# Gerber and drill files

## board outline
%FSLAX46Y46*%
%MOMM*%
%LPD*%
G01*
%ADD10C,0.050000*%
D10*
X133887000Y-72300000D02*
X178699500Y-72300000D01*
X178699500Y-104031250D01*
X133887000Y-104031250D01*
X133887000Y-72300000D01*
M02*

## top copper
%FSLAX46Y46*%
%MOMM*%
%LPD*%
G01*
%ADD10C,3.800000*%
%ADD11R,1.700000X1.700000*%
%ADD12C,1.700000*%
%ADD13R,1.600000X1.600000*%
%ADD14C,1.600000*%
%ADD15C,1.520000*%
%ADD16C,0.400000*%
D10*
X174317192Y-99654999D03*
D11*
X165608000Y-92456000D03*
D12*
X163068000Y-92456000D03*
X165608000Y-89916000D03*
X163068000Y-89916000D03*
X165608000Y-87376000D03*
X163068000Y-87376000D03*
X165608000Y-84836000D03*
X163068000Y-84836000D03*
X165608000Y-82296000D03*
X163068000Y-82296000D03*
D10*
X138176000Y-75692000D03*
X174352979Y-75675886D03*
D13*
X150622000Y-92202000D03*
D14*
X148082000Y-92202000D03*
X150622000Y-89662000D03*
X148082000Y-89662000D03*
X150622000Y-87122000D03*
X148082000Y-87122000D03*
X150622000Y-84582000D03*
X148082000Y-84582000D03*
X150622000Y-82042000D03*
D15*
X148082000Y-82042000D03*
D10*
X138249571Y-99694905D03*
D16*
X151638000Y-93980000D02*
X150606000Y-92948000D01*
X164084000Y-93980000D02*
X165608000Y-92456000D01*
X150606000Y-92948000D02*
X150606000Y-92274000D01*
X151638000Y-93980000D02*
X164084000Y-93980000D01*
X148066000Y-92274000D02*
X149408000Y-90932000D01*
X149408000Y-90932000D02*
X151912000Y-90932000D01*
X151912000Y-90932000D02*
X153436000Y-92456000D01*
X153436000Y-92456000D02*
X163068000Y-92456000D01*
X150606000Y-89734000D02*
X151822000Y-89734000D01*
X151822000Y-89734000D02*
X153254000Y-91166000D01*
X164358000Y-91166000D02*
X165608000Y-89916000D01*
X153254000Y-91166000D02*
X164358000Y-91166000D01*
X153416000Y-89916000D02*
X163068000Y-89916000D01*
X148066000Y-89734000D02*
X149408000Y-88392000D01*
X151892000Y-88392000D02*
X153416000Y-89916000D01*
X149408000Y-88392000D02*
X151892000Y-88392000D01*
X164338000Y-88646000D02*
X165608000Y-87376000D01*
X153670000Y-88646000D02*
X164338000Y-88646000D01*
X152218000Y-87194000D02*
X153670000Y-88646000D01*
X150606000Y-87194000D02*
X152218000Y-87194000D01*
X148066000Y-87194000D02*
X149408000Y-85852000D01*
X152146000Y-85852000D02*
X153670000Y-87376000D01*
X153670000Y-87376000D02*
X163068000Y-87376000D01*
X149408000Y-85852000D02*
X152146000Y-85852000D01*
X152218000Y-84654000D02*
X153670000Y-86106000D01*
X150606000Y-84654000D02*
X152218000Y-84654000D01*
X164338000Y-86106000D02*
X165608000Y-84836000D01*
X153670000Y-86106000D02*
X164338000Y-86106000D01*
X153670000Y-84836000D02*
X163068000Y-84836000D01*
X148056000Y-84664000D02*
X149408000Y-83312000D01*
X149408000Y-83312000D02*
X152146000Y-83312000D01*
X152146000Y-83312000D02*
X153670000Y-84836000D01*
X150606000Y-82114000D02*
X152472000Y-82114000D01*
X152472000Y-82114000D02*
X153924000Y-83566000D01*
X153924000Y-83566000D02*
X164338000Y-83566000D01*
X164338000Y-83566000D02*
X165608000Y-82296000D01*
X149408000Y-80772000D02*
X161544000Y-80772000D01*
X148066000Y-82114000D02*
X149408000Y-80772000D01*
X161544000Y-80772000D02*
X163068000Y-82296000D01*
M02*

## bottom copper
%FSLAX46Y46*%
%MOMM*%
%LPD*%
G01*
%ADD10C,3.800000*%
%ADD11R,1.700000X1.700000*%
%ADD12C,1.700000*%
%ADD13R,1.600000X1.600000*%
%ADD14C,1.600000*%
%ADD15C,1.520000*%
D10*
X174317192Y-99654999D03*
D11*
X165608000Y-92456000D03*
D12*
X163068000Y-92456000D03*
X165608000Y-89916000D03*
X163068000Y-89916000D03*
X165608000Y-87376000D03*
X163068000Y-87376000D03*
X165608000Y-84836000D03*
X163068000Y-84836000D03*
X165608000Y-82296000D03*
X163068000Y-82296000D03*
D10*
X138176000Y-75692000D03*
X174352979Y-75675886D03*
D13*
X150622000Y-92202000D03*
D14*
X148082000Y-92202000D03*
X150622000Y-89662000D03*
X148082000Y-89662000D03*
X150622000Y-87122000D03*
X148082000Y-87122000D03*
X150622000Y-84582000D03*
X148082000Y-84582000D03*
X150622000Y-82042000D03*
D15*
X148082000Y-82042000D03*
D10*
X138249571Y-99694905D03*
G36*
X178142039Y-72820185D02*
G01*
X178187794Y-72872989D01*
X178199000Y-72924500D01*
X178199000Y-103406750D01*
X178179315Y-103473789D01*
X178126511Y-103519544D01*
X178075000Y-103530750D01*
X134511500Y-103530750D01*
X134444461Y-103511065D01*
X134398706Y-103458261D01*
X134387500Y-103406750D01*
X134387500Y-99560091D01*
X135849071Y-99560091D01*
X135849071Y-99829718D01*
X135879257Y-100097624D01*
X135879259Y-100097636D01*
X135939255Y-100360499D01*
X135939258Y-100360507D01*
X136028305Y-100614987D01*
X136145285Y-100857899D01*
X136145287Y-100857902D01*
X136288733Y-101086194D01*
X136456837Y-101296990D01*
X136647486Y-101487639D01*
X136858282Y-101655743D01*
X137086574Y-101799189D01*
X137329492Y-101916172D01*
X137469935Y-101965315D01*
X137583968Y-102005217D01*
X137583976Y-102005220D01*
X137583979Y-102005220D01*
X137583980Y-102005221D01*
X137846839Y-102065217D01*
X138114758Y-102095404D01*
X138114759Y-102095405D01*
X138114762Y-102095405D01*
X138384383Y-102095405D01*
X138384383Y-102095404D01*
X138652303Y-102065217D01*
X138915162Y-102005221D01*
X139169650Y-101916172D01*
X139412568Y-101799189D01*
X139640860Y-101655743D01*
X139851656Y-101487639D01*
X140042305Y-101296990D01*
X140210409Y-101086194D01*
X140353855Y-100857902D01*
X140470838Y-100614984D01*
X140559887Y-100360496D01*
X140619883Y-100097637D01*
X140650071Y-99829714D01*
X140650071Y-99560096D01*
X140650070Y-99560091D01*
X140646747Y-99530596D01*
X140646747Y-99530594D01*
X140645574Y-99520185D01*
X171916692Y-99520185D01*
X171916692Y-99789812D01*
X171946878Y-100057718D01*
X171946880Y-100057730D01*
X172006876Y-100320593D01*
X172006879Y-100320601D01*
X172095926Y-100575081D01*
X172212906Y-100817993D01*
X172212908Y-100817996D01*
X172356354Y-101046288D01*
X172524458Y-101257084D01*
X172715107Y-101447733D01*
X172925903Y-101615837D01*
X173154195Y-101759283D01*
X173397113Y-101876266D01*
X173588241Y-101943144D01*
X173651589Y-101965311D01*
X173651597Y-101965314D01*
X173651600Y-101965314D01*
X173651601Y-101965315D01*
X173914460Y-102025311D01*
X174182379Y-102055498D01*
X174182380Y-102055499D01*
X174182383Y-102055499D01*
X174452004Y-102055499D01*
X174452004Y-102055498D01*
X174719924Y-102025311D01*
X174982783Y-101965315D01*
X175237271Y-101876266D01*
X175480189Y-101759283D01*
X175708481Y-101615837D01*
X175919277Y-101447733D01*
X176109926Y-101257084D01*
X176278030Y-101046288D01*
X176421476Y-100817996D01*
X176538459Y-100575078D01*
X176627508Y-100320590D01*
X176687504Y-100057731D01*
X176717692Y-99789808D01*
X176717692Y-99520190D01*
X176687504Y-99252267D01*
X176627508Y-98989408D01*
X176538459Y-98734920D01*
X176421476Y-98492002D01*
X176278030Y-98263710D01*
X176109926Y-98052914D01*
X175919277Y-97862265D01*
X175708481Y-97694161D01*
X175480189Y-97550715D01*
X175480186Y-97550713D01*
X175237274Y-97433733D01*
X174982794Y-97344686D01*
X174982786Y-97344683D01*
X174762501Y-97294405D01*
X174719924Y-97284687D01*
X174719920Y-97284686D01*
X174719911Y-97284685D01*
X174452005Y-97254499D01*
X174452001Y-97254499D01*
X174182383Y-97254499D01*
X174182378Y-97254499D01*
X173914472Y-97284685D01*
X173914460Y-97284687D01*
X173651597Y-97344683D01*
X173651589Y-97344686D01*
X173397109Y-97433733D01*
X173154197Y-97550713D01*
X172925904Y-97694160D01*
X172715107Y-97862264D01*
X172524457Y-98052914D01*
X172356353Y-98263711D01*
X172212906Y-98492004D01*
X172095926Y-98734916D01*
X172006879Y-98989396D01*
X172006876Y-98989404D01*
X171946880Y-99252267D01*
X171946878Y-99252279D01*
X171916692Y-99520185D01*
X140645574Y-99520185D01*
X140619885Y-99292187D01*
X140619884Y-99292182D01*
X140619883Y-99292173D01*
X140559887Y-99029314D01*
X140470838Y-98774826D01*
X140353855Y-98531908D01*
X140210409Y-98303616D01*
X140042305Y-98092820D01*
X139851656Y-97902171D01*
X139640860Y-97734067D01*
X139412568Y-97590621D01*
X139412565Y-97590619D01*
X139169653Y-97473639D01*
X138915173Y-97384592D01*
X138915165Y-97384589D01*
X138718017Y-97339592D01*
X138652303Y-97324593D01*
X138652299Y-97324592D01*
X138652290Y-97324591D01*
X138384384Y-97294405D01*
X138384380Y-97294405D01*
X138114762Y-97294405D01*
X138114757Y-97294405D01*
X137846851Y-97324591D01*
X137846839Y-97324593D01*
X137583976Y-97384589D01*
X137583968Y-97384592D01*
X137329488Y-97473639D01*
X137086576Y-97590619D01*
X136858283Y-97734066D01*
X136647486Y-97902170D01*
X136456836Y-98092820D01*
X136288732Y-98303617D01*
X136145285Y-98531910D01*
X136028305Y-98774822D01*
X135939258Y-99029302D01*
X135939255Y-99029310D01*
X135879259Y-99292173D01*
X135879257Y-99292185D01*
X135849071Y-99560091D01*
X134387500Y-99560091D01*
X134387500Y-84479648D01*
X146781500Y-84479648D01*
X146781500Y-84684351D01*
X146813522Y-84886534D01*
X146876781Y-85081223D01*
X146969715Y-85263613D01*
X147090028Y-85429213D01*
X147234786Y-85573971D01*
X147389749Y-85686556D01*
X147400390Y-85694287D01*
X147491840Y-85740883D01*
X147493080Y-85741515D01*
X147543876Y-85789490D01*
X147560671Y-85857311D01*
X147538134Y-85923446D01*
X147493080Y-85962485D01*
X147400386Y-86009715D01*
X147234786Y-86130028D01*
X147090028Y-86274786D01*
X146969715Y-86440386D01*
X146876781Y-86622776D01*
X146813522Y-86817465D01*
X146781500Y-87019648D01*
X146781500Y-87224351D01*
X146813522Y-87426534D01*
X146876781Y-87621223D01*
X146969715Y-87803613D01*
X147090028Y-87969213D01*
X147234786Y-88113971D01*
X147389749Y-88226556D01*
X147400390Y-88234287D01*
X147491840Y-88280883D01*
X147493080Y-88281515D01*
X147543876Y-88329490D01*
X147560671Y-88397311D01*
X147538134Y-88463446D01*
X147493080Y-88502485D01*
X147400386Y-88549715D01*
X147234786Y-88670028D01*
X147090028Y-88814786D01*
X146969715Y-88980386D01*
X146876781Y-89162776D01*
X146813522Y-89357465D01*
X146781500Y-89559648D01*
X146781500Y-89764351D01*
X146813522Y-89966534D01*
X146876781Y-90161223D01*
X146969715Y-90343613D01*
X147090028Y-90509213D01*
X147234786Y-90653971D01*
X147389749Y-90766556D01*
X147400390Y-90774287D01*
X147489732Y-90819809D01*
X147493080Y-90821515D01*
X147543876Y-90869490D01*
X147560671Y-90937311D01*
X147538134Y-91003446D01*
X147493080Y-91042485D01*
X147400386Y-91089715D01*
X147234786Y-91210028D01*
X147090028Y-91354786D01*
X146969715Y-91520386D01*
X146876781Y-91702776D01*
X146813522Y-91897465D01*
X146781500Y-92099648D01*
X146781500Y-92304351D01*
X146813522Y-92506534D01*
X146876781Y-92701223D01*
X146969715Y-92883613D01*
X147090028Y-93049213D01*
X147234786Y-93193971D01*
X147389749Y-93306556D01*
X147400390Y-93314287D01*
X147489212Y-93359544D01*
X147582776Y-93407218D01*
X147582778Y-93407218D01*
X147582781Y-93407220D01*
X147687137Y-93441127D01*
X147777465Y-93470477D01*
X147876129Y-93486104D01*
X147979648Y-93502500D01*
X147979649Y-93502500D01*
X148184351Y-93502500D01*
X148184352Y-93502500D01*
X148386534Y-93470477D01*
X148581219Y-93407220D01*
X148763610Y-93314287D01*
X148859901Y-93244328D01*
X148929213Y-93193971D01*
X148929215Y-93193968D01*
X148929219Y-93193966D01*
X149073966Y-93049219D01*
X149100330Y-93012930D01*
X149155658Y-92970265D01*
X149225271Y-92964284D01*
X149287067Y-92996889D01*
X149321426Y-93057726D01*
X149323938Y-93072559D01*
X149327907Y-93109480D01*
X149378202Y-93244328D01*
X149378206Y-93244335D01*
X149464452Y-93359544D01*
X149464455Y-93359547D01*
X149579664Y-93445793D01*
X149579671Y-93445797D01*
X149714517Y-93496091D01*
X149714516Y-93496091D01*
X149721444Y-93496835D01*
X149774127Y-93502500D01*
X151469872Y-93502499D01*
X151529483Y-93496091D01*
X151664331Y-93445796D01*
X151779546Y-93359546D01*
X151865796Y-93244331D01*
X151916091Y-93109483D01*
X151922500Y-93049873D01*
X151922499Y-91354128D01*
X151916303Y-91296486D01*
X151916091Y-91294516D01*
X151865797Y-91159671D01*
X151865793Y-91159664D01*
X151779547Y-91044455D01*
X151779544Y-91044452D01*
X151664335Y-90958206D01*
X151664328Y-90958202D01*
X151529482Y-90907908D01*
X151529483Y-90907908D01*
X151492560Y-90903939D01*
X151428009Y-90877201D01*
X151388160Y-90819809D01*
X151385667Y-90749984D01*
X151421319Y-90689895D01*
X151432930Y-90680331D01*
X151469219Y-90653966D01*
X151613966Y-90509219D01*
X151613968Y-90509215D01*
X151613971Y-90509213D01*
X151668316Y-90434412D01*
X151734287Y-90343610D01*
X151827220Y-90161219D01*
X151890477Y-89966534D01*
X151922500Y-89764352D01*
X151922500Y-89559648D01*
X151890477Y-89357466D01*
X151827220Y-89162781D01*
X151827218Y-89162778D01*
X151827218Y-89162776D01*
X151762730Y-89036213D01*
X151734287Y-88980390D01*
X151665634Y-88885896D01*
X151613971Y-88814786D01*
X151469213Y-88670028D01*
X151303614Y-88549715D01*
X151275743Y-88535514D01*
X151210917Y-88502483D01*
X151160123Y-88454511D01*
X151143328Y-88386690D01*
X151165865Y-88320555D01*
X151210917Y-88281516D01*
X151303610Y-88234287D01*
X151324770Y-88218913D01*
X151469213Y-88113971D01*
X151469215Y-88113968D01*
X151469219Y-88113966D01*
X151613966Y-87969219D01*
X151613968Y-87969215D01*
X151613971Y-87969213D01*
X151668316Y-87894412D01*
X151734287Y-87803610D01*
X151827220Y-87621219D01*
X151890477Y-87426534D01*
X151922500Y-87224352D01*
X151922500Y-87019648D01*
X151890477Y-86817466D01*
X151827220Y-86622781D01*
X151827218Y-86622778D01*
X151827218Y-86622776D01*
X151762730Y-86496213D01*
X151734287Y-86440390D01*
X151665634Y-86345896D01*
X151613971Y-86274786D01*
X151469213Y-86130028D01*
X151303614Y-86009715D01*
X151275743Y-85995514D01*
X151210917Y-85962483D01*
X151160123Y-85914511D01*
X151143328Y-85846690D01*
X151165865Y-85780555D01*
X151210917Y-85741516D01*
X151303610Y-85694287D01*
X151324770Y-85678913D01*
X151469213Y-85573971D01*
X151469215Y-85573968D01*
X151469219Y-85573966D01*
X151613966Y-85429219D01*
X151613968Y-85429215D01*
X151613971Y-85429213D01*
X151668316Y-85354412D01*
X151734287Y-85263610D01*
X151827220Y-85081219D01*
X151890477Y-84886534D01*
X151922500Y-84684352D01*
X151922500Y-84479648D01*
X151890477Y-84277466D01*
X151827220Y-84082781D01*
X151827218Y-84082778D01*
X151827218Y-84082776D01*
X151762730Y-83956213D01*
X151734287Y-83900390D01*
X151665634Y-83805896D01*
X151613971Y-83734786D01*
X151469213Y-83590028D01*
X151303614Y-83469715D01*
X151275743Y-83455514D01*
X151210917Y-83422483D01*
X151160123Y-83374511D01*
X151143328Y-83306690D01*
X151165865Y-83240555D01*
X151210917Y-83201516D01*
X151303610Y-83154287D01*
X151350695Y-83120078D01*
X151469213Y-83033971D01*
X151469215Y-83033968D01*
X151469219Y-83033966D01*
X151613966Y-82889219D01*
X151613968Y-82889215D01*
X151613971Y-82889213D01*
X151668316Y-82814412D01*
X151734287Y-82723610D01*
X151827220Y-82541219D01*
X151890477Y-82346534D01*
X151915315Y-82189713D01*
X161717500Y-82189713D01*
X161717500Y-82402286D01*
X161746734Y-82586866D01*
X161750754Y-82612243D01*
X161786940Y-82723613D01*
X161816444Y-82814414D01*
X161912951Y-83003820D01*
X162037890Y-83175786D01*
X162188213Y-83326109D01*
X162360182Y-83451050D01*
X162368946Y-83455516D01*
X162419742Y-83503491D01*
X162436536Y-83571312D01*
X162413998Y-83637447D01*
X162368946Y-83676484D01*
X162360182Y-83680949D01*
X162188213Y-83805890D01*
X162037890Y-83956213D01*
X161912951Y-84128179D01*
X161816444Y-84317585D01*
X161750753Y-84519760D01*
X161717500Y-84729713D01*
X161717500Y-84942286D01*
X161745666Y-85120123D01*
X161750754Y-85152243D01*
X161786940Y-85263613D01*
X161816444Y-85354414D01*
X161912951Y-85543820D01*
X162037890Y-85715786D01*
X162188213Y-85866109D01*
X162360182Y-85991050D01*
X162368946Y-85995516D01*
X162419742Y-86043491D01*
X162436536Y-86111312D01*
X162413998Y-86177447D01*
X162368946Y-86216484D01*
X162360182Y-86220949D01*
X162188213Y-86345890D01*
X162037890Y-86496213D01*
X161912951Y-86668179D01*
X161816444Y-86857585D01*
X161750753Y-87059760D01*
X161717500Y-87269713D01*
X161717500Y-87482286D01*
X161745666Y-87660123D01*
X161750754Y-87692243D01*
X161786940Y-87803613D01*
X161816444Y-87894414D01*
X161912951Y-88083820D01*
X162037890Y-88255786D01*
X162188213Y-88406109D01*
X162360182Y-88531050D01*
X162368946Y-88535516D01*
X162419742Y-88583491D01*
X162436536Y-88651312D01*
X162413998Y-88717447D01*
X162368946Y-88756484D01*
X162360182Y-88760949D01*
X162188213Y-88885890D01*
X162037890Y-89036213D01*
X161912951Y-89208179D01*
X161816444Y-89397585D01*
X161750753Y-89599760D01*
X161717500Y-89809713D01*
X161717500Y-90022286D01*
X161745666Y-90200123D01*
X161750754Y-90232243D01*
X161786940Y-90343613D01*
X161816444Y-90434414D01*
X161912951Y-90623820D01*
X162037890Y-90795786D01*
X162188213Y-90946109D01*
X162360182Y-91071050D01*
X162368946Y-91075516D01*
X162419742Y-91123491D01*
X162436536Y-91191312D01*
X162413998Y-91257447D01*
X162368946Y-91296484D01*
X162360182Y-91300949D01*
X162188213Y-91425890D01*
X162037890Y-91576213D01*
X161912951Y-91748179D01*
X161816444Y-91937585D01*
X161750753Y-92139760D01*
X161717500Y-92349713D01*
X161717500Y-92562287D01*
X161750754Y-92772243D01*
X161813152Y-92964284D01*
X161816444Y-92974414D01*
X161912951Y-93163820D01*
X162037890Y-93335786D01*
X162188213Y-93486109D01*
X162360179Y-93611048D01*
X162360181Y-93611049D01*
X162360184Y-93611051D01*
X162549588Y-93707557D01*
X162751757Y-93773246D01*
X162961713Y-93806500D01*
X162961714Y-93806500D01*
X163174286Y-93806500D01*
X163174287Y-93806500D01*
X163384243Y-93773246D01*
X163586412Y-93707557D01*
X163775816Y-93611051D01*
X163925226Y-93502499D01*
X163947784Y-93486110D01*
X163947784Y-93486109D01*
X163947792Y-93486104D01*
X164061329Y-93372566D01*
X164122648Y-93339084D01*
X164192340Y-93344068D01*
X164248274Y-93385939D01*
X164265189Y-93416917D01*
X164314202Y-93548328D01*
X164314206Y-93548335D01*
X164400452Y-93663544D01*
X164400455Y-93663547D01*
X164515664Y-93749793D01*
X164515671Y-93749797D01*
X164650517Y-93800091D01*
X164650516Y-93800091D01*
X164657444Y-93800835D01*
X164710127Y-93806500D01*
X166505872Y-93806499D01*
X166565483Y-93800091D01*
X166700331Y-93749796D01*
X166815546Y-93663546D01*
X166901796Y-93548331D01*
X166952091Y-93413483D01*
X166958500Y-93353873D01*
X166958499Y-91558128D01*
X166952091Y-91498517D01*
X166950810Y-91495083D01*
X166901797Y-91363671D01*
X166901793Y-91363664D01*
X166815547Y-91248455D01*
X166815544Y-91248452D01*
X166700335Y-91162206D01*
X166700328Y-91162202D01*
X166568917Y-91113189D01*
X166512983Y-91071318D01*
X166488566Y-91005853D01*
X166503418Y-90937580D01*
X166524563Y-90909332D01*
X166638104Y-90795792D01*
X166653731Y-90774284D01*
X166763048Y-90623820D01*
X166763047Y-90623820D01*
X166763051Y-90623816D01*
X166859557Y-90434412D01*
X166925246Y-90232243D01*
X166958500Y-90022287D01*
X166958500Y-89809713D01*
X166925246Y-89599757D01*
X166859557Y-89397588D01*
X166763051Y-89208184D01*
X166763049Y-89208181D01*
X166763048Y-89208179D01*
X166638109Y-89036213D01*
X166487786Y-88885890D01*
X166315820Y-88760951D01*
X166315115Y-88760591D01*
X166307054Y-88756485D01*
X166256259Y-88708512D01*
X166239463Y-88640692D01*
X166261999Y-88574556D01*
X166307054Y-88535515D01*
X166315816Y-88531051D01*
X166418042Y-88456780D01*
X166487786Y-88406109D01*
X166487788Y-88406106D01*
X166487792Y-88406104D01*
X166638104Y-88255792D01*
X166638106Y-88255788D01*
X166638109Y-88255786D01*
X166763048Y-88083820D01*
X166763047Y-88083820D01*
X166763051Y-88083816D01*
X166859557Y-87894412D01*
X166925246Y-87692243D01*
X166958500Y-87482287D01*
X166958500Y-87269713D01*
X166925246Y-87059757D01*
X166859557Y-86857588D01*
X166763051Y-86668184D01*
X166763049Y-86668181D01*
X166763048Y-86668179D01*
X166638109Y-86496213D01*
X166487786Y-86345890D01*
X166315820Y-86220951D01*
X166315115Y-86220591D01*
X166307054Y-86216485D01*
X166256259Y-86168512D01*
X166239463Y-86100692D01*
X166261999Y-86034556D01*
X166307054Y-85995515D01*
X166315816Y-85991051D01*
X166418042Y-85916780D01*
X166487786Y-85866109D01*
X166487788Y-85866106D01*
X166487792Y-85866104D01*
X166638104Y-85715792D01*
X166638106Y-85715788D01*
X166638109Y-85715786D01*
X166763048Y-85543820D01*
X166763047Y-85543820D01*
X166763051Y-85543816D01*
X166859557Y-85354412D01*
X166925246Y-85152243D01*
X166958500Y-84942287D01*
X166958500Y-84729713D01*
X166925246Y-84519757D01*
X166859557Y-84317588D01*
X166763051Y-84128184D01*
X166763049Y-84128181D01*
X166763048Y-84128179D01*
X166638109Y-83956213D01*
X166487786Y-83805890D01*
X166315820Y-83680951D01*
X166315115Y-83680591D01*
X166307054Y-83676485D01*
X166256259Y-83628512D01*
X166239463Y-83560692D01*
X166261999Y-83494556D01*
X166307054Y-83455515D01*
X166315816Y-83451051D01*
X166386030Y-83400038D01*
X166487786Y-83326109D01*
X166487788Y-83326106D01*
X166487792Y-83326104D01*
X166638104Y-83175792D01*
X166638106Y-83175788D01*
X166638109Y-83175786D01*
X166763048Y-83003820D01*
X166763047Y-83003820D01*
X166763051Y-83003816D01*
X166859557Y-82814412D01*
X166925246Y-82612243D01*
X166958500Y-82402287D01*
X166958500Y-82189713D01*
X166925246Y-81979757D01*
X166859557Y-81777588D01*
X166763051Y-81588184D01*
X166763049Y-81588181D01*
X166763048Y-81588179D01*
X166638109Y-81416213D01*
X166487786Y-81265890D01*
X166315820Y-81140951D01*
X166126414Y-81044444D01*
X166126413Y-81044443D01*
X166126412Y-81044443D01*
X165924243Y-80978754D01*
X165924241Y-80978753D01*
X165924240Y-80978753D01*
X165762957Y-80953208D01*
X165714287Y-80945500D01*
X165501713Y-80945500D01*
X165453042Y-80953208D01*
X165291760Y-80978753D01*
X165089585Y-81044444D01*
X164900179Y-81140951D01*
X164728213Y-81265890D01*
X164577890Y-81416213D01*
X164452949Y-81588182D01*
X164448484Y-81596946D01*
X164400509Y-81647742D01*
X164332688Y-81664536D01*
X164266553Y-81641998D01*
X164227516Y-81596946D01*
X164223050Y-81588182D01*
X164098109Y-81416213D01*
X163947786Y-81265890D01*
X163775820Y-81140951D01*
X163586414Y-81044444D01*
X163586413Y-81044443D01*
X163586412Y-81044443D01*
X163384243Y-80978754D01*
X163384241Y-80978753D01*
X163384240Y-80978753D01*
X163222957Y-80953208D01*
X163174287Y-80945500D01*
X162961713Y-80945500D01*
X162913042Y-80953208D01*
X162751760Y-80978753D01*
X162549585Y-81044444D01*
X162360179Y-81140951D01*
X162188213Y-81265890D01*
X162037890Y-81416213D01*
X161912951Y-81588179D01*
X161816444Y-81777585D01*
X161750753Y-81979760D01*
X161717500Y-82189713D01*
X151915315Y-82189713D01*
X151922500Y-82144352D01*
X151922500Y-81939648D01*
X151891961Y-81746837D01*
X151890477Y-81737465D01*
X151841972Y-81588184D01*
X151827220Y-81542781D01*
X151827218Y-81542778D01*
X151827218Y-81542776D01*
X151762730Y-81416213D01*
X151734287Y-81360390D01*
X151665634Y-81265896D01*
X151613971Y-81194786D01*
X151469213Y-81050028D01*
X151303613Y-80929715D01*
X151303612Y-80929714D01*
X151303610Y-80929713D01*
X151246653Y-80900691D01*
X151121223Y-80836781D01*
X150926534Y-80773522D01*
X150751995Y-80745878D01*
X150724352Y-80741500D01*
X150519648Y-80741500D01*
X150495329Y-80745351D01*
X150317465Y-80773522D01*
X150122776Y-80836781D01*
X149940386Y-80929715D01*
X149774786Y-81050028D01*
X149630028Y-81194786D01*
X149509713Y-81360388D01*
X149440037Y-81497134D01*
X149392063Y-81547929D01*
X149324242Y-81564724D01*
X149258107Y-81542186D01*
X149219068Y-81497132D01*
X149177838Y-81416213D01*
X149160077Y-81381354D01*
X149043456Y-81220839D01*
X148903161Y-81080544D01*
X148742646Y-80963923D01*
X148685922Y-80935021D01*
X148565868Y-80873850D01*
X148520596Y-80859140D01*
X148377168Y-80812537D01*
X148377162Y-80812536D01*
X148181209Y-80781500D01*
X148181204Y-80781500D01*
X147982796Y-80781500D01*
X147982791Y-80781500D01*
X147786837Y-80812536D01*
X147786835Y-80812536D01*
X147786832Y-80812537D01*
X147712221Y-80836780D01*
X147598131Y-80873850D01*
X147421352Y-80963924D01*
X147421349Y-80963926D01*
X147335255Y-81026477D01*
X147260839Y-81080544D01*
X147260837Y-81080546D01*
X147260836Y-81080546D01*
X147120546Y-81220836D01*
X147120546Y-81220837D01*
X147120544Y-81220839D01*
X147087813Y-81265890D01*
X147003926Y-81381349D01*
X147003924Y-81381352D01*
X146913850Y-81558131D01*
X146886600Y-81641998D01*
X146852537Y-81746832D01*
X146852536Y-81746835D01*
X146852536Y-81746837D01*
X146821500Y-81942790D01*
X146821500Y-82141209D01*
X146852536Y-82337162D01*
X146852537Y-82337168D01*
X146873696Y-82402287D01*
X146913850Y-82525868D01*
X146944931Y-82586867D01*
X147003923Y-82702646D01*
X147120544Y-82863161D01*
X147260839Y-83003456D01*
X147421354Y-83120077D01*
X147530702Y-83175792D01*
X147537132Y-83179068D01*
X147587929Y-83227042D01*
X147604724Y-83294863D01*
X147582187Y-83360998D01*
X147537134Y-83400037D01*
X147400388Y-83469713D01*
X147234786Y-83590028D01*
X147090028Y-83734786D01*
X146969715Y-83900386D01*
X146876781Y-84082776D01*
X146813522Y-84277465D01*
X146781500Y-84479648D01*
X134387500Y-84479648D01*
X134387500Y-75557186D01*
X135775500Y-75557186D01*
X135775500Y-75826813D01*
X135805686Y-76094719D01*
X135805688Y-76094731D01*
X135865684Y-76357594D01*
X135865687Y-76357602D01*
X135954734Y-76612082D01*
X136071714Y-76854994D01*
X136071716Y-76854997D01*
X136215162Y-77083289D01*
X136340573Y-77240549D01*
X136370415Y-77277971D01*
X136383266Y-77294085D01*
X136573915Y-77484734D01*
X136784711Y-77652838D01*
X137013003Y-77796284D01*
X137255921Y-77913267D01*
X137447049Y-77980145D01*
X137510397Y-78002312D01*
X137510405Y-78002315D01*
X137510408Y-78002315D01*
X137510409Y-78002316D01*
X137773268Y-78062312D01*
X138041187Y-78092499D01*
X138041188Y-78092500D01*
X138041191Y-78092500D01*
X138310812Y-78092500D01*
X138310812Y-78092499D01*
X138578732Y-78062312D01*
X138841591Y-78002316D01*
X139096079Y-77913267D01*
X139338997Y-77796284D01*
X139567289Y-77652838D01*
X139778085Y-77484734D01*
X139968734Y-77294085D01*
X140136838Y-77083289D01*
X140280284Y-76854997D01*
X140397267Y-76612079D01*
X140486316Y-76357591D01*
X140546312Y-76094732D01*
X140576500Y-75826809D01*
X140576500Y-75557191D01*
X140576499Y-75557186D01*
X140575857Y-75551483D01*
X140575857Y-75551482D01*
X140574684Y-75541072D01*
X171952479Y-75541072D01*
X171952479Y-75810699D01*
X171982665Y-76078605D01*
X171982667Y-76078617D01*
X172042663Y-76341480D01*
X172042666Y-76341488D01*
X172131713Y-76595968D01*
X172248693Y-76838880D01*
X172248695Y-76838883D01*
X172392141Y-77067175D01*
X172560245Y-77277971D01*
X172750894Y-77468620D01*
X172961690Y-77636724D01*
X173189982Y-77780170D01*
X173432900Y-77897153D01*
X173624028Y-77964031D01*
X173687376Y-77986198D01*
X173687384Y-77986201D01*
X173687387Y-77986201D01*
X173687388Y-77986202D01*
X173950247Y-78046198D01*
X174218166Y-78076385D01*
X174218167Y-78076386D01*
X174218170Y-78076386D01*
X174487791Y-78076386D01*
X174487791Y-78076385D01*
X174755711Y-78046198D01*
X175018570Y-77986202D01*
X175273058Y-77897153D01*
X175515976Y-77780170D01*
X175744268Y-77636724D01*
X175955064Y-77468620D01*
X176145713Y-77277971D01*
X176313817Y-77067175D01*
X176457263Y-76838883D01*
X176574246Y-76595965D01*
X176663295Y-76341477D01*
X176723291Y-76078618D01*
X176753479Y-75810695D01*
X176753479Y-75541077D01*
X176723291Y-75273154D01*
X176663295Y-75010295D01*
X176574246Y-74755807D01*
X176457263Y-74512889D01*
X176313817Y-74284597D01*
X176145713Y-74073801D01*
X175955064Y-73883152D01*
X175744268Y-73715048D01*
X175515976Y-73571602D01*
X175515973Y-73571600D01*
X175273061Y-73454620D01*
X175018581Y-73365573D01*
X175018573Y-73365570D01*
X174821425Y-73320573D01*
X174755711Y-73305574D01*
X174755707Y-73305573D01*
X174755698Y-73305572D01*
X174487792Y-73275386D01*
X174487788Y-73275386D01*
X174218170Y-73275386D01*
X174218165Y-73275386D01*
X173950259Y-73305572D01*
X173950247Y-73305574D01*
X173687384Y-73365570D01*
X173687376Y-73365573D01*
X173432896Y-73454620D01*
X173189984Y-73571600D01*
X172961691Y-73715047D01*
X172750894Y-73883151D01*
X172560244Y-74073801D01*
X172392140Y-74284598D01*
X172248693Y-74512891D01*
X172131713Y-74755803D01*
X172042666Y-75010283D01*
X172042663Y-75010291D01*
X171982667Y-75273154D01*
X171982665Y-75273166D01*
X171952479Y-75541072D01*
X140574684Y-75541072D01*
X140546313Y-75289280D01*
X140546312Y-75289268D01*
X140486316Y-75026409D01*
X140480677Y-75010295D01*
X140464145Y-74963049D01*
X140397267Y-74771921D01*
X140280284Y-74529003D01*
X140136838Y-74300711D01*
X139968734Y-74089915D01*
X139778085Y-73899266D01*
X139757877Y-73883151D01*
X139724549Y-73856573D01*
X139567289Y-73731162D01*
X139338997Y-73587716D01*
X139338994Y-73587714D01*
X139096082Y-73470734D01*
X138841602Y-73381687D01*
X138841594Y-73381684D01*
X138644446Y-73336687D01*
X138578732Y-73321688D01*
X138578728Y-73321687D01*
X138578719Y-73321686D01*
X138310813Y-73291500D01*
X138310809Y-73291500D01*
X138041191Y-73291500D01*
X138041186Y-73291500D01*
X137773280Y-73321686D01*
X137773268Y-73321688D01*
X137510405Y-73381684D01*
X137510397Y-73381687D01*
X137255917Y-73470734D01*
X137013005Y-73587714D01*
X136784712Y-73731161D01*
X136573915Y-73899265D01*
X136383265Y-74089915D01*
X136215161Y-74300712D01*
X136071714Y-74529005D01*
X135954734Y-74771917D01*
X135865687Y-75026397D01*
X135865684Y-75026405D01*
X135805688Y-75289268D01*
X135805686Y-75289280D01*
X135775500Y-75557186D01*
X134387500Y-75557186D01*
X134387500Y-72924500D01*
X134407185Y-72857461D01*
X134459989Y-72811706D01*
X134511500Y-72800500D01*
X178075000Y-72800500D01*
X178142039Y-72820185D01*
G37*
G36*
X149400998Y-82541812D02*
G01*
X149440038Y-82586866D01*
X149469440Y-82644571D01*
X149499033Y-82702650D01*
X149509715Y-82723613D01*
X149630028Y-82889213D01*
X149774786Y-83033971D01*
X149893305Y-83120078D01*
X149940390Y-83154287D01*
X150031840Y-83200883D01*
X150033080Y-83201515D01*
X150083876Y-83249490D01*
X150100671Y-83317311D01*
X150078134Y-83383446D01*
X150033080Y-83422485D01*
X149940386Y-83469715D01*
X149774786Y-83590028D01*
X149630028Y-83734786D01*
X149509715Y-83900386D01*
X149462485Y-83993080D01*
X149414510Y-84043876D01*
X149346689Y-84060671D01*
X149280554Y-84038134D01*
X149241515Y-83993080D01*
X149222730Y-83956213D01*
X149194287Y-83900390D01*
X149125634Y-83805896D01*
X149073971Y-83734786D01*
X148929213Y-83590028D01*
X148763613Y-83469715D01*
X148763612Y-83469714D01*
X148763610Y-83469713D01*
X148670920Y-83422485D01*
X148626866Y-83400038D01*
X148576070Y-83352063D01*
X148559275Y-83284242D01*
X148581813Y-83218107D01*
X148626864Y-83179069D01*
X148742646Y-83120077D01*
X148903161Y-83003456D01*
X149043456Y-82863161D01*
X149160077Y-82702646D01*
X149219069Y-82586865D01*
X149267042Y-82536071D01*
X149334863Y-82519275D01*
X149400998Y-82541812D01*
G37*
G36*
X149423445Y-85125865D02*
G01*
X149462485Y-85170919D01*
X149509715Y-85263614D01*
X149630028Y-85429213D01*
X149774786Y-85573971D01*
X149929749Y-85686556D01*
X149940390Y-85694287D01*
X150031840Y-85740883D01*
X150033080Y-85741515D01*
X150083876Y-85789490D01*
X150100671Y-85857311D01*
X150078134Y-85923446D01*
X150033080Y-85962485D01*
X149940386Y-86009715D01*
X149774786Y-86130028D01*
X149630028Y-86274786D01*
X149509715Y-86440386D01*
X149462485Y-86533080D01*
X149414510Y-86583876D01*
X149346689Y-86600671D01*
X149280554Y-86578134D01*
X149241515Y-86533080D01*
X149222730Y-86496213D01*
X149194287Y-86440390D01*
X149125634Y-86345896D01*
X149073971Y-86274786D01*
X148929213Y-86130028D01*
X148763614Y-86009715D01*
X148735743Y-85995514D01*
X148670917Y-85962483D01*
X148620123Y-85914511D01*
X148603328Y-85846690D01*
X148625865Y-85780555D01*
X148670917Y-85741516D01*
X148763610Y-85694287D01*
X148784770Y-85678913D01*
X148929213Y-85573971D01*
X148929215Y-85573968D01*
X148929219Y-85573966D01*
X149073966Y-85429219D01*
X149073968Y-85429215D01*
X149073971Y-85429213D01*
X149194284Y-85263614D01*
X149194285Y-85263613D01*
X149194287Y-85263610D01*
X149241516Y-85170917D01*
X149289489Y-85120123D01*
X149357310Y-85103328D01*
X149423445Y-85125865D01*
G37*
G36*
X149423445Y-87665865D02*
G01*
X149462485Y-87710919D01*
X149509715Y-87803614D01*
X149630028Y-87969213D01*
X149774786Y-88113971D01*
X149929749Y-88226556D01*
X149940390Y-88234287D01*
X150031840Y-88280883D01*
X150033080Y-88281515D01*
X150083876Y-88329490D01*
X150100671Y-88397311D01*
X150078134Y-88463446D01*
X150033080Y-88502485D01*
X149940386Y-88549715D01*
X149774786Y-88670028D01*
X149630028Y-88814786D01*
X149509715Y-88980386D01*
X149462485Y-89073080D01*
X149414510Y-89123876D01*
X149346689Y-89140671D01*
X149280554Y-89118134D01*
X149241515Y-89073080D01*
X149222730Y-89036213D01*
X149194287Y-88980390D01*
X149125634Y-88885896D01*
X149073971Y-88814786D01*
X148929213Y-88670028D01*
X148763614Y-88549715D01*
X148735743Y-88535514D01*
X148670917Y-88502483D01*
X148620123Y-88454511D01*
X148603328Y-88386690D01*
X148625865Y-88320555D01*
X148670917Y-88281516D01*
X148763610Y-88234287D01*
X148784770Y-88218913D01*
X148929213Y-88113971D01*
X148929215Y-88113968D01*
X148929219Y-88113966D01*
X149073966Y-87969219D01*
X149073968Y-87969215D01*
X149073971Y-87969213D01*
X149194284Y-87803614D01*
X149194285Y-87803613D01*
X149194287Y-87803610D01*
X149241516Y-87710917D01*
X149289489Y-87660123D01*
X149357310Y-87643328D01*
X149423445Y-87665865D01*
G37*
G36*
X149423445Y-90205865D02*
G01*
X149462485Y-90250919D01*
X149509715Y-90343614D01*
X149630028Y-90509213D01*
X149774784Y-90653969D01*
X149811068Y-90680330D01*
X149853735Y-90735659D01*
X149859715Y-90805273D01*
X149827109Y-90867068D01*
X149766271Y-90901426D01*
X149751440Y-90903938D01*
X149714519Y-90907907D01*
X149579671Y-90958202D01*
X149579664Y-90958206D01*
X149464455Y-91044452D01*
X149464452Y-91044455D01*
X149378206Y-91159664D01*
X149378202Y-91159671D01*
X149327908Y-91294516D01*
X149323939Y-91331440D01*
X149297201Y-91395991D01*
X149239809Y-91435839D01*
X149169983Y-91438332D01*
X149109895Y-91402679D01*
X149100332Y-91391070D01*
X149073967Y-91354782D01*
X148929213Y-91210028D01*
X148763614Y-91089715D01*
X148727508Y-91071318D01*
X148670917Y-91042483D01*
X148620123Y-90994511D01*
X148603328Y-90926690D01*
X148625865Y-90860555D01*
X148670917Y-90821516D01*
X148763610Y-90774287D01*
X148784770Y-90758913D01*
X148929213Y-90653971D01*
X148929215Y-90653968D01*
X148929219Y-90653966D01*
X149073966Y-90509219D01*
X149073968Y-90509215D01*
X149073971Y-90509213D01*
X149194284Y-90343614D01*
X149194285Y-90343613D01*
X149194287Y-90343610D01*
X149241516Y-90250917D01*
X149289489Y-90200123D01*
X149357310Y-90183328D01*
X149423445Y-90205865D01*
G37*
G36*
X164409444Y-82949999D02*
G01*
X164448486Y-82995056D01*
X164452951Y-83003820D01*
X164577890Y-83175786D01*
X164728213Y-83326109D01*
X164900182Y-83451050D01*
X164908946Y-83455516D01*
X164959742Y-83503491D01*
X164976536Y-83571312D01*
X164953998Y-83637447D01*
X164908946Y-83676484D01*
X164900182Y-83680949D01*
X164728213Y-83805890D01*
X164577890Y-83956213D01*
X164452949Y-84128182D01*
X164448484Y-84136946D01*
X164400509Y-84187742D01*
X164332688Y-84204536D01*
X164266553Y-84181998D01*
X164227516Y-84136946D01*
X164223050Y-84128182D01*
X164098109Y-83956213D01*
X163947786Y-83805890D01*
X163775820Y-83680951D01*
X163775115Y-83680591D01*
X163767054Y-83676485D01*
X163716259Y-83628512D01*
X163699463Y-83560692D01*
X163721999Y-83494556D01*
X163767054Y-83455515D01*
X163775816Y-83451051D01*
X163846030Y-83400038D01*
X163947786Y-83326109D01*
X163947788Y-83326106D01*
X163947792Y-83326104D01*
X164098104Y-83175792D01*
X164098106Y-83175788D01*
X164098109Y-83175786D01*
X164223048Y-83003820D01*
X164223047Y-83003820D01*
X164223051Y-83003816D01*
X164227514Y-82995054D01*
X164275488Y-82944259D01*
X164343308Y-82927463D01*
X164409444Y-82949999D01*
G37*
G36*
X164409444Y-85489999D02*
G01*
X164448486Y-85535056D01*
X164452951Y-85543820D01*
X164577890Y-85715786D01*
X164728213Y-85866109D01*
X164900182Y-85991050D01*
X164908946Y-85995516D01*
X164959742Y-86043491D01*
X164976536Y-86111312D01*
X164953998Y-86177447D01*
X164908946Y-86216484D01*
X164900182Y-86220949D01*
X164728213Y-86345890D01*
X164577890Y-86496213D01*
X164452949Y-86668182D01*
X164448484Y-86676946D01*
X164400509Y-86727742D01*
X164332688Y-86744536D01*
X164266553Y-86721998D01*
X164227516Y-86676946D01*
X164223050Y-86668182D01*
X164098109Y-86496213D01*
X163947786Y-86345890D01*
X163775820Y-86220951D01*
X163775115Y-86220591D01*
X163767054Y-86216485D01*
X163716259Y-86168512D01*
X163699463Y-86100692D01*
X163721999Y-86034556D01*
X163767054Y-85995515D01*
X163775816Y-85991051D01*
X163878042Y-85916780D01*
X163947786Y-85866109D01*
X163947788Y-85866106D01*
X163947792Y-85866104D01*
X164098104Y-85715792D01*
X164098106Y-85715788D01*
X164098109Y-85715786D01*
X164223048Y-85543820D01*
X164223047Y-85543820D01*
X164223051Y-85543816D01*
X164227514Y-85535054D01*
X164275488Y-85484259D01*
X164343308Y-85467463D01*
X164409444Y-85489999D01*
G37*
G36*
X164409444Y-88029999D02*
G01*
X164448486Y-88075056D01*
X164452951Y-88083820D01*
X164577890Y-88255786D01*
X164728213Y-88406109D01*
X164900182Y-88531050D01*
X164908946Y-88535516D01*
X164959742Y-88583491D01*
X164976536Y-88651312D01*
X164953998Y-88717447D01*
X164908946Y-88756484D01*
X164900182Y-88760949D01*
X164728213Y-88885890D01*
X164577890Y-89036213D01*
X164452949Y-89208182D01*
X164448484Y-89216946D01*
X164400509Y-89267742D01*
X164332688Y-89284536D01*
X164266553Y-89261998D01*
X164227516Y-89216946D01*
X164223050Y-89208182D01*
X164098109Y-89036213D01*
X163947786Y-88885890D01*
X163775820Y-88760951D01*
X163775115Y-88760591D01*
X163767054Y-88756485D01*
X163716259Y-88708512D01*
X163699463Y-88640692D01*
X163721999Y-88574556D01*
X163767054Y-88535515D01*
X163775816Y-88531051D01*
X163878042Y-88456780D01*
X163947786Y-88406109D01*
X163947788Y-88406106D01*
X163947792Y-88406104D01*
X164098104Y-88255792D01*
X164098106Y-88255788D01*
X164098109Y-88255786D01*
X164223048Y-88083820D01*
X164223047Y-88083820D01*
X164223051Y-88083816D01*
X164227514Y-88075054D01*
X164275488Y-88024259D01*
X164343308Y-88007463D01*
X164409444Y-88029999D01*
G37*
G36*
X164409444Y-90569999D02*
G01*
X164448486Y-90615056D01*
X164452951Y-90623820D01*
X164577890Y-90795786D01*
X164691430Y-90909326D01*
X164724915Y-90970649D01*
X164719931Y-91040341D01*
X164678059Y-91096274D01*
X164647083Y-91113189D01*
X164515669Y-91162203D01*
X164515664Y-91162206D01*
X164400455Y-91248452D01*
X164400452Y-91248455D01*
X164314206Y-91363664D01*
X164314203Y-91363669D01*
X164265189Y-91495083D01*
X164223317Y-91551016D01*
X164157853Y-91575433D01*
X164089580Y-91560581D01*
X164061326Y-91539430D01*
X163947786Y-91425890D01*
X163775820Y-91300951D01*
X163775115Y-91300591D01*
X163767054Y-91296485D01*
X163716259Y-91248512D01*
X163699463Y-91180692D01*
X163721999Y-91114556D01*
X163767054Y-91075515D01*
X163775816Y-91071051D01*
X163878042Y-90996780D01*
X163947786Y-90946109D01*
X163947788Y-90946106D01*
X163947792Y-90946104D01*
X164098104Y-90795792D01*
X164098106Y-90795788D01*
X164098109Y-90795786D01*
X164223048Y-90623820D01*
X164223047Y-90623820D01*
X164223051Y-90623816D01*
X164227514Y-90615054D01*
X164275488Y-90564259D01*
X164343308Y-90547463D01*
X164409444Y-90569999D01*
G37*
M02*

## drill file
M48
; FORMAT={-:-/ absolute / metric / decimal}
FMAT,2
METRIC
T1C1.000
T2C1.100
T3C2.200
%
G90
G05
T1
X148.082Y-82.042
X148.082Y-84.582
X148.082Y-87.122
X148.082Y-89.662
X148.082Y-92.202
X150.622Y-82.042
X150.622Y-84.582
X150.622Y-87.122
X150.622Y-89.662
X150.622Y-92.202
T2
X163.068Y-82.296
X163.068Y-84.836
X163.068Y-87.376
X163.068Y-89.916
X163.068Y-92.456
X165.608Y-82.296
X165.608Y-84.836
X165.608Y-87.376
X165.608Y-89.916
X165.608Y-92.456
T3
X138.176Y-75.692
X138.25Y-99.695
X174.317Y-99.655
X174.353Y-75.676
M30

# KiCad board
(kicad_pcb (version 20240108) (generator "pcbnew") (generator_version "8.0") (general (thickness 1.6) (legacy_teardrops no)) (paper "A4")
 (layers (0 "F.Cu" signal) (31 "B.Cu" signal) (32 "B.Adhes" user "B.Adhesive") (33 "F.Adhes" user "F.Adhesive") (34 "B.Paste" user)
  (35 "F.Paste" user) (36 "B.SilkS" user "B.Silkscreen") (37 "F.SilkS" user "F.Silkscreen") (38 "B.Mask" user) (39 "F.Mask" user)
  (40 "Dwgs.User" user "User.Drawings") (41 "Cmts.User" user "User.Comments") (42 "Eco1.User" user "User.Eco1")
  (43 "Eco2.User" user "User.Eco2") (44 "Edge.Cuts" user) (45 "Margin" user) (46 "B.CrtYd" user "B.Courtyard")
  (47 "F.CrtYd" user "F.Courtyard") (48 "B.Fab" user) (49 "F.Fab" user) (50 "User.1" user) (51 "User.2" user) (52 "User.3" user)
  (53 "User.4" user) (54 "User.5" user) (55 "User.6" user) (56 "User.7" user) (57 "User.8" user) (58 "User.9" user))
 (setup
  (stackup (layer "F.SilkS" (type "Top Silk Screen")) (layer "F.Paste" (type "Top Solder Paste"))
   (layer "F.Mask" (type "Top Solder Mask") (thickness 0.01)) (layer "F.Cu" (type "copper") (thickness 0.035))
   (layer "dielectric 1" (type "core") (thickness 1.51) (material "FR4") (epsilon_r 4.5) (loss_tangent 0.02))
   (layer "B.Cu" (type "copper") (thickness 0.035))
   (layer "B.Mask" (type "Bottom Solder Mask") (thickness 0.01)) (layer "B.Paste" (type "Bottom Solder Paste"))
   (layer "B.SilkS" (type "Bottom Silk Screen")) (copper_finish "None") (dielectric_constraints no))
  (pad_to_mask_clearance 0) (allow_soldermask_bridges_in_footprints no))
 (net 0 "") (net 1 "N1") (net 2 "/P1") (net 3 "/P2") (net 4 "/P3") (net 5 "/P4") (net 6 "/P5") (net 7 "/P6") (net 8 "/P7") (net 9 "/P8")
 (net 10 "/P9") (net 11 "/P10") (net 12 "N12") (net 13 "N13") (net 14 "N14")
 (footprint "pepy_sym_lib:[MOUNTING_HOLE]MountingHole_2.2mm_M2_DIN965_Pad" (layer "F.Cu") (at 174.317192 99.654999)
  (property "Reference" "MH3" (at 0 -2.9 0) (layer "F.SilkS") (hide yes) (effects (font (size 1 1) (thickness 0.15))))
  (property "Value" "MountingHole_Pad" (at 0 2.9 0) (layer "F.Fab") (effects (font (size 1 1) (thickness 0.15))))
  (pad "1" thru_hole circle (at 0 0) (size 3.8 3.8) (drill 2.2) (layers "*.Cu" "*.Mask") (remove_unused_layers no) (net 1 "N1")))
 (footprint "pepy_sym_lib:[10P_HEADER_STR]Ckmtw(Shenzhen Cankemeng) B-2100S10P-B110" (layer "F.Cu") (at 164.338 87.376 90)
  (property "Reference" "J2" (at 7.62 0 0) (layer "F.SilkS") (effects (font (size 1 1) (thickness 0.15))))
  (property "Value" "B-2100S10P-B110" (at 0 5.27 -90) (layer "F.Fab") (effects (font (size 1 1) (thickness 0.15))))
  (pad "1" thru_hole rect (at -5.08 1.27 90) (size 1.7 1.7) (drill 1.100023) (layers "*.Cu" "*.Mask") (remove_unused_layers no)
   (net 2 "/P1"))
  (pad "2" thru_hole circle (at -5.08 -1.27 90) (size 1.7 1.7) (drill 1.100023) (layers "*.Cu" "*.Mask") (remove_unused_layers no)
   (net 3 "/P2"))
  (pad "3" thru_hole circle (at -2.54 1.27 90) (size 1.7 1.7) (drill 1.100023) (layers "*.Cu" "*.Mask") (remove_unused_layers no)
   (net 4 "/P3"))
  (pad "4" thru_hole circle (at -2.54 -1.27 90) (size 1.7 1.7) (drill 1.100023) (layers "*.Cu" "*.Mask") (remove_unused_layers no)
   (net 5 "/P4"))
  (pad "5" thru_hole circle (at 0 1.27 90) (size 1.7 1.7) (drill 1.100023) (layers "*.Cu" "*.Mask") (remove_unused_layers no) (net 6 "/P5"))
  (pad "6" thru_hole circle (at 0 -1.27 90) (size 1.7 1.7) (drill 1.100023) (layers "*.Cu" "*.Mask") (remove_unused_layers no) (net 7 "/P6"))
  (pad "7" thru_hole circle (at 2.54 1.27 90) (size 1.7 1.7) (drill 1.100023) (layers "*.Cu" "*.Mask") (remove_unused_layers no)
   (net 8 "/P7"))
  (pad "8" thru_hole circle (at 2.54 -1.27 90) (size 1.7 1.7) (drill 1.100023) (layers "*.Cu" "*.Mask") (remove_unused_layers no)
   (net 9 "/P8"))
  (pad "9" thru_hole circle (at 5.08 1.27 90) (size 1.7 1.7) (drill 1.100023) (layers "*.Cu" "*.Mask") (remove_unused_layers no)
   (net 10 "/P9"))
  (pad "10" thru_hole circle (at 5.08 -1.27 90) (size 1.7 1.7) (drill 1.100023) (layers "*.Cu" "*.Mask") (remove_unused_layers no)
   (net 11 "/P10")))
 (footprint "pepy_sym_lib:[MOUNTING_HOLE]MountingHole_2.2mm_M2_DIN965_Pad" (layer "F.Cu") (at 138.176 75.692)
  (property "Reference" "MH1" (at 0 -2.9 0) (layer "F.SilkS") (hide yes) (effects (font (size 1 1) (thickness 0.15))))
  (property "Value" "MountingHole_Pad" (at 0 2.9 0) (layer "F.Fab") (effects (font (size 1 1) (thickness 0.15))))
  (pad "1" thru_hole circle (at 0 0) (size 3.8 3.8) (drill 2.2) (layers "*.Cu" "*.Mask") (remove_unused_layers no) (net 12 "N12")))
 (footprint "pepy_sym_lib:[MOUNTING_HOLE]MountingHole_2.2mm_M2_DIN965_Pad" (layer "F.Cu") (at 174.352979 75.675886)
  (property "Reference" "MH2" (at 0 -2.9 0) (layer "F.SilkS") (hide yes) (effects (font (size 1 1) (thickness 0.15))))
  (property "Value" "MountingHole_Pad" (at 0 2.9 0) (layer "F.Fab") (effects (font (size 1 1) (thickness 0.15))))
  (pad "1" thru_hole circle (at 0 0) (size 3.8 3.8) (drill 2.2) (layers "*.Cu" "*.Mask") (remove_unused_layers no) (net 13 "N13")))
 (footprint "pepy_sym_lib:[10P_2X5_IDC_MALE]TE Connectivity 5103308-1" (layer "F.Cu") (at 149.352 87.122 -90)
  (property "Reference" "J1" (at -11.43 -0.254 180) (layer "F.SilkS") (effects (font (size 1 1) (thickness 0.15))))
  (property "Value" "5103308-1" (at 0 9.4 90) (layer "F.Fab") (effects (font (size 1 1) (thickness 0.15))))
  (pad "1" thru_hole rect (at 5.08 -1.27 270) (size 1.6 1.6) (drill 0.999998) (layers "*.Cu" "*.Mask") (remove_unused_layers no)
   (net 2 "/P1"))
  (pad "2" thru_hole circle (at 5.08 1.27 270) (size 1.6 1.6) (drill 0.999998) (layers "*.Cu" "*.Mask") (remove_unused_layers no)
   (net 3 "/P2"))
  (pad "3" thru_hole circle (at 2.54 -1.27 270) (size 1.6 1.6) (drill 0.999998) (layers "*.Cu" "*.Mask") (remove_unused_layers no)
   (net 4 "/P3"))
  (pad "4" thru_hole circle (at 2.54 1.27 270) (size 1.6 1.6) (drill 0.999998) (layers "*.Cu" "*.Mask") (remove_unused_layers no)
   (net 5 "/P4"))
  (pad "5" thru_hole circle (at 0 -1.27 270) (size 1.6 1.6) (drill 0.999998) (layers "*.Cu" "*.Mask") (remove_unused_layers no)
   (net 6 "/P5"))
  (pad "6" thru_hole circle (at 0 1.27 270) (size 1.6 1.6) (drill 0.999998) (layers "*.Cu" "*.Mask") (remove_unused_layers no) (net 7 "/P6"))
  (pad "7" thru_hole circle (at -2.54 -1.27 270) (size 1.6 1.6) (drill 0.999998) (layers "*.Cu" "*.Mask") (remove_unused_layers no)
   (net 8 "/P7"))
  (pad "8" thru_hole circle (at -2.54 1.27 270) (size 1.6 1.6) (drill 0.999998) (layers "*.Cu" "*.Mask") (remove_unused_layers no)
   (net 9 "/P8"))
  (pad "9" thru_hole circle (at -5.08 -1.27 270) (size 1.6 1.6) (drill 0.999998) (layers "*.Cu" "*.Mask") (remove_unused_layers no)
   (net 10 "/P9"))
  (pad "10" thru_hole circle (at -5.08 1.27 270) (size 1.52 1.52) (drill 0.999998) (layers "*.Cu" "*.Mask") (remove_unused_layers no)
   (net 11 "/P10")))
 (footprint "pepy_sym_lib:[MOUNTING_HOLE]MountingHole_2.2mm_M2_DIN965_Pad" (layer "F.Cu") (at 138.249571 99.694905)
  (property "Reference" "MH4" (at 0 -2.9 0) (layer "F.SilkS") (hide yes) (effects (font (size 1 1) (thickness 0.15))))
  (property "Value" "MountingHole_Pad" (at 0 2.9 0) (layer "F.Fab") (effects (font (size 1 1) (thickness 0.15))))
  (pad "1" thru_hole circle (at 0 0) (size 3.8 3.8) (drill 2.2) (layers "*.Cu" "*.Mask") (remove_unused_layers no) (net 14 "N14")))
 (gr_rect (start 133.887 72.3) (end 178.6995 104.03125) (stroke (width 0.05) (type default)) (fill none) (layer "Edge.Cuts"))
 (segment (start 151.638 93.98) (end 150.606 92.948) (width 0.4) (layer "F.Cu") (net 2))
 (segment (start 164.084 93.98) (end 165.608 92.456) (width 0.4) (layer "F.Cu") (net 2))
 (segment (start 150.606 92.948) (end 150.606 92.274) (width 0.4) (layer "F.Cu") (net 2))
 (segment (start 151.638 93.98) (end 164.084 93.98) (width 0.4) (layer "F.Cu") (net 2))
 (segment (start 148.066 92.274) (end 149.408 90.932) (width 0.4) (layer "F.Cu") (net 3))
 (segment (start 149.408 90.932) (end 151.912 90.932) (width 0.4) (layer "F.Cu") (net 3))
 (segment (start 151.912 90.932) (end 153.436 92.456) (width 0.4) (layer "F.Cu") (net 3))
 (segment (start 153.436 92.456) (end 163.068 92.456) (width 0.4) (layer "F.Cu") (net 3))
 (segment (start 150.606 89.734) (end 151.822 89.734) (width 0.4) (layer "F.Cu") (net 4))
 (segment (start 151.822 89.734) (end 153.254 91.166) (width 0.4) (layer "F.Cu") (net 4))
 (segment (start 164.358 91.166) (end 165.608 89.916) (width 0.4) (layer "F.Cu") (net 4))
 (segment (start 153.254 91.166) (end 164.358 91.166) (width 0.4) (layer "F.Cu") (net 4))
 (segment (start 153.416 89.916) (end 163.068 89.916) (width 0.4) (layer "F.Cu") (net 5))
 (segment (start 148.066 89.734) (end 149.408 88.392) (width 0.4) (layer "F.Cu") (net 5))
 (segment (start 151.892 88.392) (end 153.416 89.916) (width 0.4) (layer "F.Cu") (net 5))
 (segment (start 149.408 88.392) (end 151.892 88.392) (width 0.4) (layer "F.Cu") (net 5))
 (segment (start 164.338 88.646) (end 165.608 87.376) (width 0.4) (layer "F.Cu") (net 6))
 (segment (start 153.67 88.646) (end 164.338 88.646) (width 0.4) (layer "F.Cu") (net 6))
 (segment (start 152.218 87.194) (end 153.67 88.646) (width 0.4) (layer "F.Cu") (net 6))
 (segment (start 150.606 87.194) (end 152.218 87.194) (width 0.4) (layer "F.Cu") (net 6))
 (segment (start 148.066 87.194) (end 149.408 85.852) (width 0.4) (layer "F.Cu") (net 7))
 (segment (start 152.146 85.852) (end 153.67 87.376) (width 0.4) (layer "F.Cu") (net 7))
 (segment (start 153.67 87.376) (end 163.068 87.376) (width 0.4) (layer "F.Cu") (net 7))
 (segment (start 149.408 85.852) (end 152.146 85.852) (width 0.4) (layer "F.Cu") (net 7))
 (segment (start 152.218 84.654) (end 153.67 86.106) (width 0.4) (layer "F.Cu") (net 8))
 (segment (start 150.606 84.654) (end 152.218 84.654) (width 0.4) (layer "F.Cu") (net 8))
 (segment (start 164.338 86.106) (end 165.608 84.836) (width 0.4) (layer "F.Cu") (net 8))
 (segment (start 153.67 86.106) (end 164.338 86.106) (width 0.4) (layer "F.Cu") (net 8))
 (segment (start 153.67 84.836) (end 163.068 84.836) (width 0.4) (layer "F.Cu") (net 9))
 (segment (start 148.056 84.664) (end 149.408 83.312) (width 0.4) (layer "F.Cu") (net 9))
 (segment (start 149.408 83.312) (end 152.146 83.312) (width 0.4) (layer "F.Cu") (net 9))
 (segment (start 152.146 83.312) (end 153.67 84.836) (width 0.4) (layer "F.Cu") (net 9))
 (segment (start 150.606 82.114) (end 152.472 82.114) (width 0.4) (layer "F.Cu") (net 10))
 (segment (start 152.472 82.114) (end 153.924 83.566) (width 0.4) (layer "F.Cu") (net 10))
 (segment (start 153.924 83.566) (end 164.338 83.566) (width 0.4) (layer "F.Cu") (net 10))
 (segment (start 164.338 83.566) (end 165.608 82.296) (width 0.4) (layer "F.Cu") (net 10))
 (segment (start 149.408 80.772) (end 161.544 80.772) (width 0.4) (layer "F.Cu") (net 11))
 (segment (start 148.066 82.114) (end 149.408 80.772) (width 0.4) (layer "F.Cu") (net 11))
 (segment (start 161.544 80.772) (end 163.068 82.296) (width 0.4) (layer "F.Cu") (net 11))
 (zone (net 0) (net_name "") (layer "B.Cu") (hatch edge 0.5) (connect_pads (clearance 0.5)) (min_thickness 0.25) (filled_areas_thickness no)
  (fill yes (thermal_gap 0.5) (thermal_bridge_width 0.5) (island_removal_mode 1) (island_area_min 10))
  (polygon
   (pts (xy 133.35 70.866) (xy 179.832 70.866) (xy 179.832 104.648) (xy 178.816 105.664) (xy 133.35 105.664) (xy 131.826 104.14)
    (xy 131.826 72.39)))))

